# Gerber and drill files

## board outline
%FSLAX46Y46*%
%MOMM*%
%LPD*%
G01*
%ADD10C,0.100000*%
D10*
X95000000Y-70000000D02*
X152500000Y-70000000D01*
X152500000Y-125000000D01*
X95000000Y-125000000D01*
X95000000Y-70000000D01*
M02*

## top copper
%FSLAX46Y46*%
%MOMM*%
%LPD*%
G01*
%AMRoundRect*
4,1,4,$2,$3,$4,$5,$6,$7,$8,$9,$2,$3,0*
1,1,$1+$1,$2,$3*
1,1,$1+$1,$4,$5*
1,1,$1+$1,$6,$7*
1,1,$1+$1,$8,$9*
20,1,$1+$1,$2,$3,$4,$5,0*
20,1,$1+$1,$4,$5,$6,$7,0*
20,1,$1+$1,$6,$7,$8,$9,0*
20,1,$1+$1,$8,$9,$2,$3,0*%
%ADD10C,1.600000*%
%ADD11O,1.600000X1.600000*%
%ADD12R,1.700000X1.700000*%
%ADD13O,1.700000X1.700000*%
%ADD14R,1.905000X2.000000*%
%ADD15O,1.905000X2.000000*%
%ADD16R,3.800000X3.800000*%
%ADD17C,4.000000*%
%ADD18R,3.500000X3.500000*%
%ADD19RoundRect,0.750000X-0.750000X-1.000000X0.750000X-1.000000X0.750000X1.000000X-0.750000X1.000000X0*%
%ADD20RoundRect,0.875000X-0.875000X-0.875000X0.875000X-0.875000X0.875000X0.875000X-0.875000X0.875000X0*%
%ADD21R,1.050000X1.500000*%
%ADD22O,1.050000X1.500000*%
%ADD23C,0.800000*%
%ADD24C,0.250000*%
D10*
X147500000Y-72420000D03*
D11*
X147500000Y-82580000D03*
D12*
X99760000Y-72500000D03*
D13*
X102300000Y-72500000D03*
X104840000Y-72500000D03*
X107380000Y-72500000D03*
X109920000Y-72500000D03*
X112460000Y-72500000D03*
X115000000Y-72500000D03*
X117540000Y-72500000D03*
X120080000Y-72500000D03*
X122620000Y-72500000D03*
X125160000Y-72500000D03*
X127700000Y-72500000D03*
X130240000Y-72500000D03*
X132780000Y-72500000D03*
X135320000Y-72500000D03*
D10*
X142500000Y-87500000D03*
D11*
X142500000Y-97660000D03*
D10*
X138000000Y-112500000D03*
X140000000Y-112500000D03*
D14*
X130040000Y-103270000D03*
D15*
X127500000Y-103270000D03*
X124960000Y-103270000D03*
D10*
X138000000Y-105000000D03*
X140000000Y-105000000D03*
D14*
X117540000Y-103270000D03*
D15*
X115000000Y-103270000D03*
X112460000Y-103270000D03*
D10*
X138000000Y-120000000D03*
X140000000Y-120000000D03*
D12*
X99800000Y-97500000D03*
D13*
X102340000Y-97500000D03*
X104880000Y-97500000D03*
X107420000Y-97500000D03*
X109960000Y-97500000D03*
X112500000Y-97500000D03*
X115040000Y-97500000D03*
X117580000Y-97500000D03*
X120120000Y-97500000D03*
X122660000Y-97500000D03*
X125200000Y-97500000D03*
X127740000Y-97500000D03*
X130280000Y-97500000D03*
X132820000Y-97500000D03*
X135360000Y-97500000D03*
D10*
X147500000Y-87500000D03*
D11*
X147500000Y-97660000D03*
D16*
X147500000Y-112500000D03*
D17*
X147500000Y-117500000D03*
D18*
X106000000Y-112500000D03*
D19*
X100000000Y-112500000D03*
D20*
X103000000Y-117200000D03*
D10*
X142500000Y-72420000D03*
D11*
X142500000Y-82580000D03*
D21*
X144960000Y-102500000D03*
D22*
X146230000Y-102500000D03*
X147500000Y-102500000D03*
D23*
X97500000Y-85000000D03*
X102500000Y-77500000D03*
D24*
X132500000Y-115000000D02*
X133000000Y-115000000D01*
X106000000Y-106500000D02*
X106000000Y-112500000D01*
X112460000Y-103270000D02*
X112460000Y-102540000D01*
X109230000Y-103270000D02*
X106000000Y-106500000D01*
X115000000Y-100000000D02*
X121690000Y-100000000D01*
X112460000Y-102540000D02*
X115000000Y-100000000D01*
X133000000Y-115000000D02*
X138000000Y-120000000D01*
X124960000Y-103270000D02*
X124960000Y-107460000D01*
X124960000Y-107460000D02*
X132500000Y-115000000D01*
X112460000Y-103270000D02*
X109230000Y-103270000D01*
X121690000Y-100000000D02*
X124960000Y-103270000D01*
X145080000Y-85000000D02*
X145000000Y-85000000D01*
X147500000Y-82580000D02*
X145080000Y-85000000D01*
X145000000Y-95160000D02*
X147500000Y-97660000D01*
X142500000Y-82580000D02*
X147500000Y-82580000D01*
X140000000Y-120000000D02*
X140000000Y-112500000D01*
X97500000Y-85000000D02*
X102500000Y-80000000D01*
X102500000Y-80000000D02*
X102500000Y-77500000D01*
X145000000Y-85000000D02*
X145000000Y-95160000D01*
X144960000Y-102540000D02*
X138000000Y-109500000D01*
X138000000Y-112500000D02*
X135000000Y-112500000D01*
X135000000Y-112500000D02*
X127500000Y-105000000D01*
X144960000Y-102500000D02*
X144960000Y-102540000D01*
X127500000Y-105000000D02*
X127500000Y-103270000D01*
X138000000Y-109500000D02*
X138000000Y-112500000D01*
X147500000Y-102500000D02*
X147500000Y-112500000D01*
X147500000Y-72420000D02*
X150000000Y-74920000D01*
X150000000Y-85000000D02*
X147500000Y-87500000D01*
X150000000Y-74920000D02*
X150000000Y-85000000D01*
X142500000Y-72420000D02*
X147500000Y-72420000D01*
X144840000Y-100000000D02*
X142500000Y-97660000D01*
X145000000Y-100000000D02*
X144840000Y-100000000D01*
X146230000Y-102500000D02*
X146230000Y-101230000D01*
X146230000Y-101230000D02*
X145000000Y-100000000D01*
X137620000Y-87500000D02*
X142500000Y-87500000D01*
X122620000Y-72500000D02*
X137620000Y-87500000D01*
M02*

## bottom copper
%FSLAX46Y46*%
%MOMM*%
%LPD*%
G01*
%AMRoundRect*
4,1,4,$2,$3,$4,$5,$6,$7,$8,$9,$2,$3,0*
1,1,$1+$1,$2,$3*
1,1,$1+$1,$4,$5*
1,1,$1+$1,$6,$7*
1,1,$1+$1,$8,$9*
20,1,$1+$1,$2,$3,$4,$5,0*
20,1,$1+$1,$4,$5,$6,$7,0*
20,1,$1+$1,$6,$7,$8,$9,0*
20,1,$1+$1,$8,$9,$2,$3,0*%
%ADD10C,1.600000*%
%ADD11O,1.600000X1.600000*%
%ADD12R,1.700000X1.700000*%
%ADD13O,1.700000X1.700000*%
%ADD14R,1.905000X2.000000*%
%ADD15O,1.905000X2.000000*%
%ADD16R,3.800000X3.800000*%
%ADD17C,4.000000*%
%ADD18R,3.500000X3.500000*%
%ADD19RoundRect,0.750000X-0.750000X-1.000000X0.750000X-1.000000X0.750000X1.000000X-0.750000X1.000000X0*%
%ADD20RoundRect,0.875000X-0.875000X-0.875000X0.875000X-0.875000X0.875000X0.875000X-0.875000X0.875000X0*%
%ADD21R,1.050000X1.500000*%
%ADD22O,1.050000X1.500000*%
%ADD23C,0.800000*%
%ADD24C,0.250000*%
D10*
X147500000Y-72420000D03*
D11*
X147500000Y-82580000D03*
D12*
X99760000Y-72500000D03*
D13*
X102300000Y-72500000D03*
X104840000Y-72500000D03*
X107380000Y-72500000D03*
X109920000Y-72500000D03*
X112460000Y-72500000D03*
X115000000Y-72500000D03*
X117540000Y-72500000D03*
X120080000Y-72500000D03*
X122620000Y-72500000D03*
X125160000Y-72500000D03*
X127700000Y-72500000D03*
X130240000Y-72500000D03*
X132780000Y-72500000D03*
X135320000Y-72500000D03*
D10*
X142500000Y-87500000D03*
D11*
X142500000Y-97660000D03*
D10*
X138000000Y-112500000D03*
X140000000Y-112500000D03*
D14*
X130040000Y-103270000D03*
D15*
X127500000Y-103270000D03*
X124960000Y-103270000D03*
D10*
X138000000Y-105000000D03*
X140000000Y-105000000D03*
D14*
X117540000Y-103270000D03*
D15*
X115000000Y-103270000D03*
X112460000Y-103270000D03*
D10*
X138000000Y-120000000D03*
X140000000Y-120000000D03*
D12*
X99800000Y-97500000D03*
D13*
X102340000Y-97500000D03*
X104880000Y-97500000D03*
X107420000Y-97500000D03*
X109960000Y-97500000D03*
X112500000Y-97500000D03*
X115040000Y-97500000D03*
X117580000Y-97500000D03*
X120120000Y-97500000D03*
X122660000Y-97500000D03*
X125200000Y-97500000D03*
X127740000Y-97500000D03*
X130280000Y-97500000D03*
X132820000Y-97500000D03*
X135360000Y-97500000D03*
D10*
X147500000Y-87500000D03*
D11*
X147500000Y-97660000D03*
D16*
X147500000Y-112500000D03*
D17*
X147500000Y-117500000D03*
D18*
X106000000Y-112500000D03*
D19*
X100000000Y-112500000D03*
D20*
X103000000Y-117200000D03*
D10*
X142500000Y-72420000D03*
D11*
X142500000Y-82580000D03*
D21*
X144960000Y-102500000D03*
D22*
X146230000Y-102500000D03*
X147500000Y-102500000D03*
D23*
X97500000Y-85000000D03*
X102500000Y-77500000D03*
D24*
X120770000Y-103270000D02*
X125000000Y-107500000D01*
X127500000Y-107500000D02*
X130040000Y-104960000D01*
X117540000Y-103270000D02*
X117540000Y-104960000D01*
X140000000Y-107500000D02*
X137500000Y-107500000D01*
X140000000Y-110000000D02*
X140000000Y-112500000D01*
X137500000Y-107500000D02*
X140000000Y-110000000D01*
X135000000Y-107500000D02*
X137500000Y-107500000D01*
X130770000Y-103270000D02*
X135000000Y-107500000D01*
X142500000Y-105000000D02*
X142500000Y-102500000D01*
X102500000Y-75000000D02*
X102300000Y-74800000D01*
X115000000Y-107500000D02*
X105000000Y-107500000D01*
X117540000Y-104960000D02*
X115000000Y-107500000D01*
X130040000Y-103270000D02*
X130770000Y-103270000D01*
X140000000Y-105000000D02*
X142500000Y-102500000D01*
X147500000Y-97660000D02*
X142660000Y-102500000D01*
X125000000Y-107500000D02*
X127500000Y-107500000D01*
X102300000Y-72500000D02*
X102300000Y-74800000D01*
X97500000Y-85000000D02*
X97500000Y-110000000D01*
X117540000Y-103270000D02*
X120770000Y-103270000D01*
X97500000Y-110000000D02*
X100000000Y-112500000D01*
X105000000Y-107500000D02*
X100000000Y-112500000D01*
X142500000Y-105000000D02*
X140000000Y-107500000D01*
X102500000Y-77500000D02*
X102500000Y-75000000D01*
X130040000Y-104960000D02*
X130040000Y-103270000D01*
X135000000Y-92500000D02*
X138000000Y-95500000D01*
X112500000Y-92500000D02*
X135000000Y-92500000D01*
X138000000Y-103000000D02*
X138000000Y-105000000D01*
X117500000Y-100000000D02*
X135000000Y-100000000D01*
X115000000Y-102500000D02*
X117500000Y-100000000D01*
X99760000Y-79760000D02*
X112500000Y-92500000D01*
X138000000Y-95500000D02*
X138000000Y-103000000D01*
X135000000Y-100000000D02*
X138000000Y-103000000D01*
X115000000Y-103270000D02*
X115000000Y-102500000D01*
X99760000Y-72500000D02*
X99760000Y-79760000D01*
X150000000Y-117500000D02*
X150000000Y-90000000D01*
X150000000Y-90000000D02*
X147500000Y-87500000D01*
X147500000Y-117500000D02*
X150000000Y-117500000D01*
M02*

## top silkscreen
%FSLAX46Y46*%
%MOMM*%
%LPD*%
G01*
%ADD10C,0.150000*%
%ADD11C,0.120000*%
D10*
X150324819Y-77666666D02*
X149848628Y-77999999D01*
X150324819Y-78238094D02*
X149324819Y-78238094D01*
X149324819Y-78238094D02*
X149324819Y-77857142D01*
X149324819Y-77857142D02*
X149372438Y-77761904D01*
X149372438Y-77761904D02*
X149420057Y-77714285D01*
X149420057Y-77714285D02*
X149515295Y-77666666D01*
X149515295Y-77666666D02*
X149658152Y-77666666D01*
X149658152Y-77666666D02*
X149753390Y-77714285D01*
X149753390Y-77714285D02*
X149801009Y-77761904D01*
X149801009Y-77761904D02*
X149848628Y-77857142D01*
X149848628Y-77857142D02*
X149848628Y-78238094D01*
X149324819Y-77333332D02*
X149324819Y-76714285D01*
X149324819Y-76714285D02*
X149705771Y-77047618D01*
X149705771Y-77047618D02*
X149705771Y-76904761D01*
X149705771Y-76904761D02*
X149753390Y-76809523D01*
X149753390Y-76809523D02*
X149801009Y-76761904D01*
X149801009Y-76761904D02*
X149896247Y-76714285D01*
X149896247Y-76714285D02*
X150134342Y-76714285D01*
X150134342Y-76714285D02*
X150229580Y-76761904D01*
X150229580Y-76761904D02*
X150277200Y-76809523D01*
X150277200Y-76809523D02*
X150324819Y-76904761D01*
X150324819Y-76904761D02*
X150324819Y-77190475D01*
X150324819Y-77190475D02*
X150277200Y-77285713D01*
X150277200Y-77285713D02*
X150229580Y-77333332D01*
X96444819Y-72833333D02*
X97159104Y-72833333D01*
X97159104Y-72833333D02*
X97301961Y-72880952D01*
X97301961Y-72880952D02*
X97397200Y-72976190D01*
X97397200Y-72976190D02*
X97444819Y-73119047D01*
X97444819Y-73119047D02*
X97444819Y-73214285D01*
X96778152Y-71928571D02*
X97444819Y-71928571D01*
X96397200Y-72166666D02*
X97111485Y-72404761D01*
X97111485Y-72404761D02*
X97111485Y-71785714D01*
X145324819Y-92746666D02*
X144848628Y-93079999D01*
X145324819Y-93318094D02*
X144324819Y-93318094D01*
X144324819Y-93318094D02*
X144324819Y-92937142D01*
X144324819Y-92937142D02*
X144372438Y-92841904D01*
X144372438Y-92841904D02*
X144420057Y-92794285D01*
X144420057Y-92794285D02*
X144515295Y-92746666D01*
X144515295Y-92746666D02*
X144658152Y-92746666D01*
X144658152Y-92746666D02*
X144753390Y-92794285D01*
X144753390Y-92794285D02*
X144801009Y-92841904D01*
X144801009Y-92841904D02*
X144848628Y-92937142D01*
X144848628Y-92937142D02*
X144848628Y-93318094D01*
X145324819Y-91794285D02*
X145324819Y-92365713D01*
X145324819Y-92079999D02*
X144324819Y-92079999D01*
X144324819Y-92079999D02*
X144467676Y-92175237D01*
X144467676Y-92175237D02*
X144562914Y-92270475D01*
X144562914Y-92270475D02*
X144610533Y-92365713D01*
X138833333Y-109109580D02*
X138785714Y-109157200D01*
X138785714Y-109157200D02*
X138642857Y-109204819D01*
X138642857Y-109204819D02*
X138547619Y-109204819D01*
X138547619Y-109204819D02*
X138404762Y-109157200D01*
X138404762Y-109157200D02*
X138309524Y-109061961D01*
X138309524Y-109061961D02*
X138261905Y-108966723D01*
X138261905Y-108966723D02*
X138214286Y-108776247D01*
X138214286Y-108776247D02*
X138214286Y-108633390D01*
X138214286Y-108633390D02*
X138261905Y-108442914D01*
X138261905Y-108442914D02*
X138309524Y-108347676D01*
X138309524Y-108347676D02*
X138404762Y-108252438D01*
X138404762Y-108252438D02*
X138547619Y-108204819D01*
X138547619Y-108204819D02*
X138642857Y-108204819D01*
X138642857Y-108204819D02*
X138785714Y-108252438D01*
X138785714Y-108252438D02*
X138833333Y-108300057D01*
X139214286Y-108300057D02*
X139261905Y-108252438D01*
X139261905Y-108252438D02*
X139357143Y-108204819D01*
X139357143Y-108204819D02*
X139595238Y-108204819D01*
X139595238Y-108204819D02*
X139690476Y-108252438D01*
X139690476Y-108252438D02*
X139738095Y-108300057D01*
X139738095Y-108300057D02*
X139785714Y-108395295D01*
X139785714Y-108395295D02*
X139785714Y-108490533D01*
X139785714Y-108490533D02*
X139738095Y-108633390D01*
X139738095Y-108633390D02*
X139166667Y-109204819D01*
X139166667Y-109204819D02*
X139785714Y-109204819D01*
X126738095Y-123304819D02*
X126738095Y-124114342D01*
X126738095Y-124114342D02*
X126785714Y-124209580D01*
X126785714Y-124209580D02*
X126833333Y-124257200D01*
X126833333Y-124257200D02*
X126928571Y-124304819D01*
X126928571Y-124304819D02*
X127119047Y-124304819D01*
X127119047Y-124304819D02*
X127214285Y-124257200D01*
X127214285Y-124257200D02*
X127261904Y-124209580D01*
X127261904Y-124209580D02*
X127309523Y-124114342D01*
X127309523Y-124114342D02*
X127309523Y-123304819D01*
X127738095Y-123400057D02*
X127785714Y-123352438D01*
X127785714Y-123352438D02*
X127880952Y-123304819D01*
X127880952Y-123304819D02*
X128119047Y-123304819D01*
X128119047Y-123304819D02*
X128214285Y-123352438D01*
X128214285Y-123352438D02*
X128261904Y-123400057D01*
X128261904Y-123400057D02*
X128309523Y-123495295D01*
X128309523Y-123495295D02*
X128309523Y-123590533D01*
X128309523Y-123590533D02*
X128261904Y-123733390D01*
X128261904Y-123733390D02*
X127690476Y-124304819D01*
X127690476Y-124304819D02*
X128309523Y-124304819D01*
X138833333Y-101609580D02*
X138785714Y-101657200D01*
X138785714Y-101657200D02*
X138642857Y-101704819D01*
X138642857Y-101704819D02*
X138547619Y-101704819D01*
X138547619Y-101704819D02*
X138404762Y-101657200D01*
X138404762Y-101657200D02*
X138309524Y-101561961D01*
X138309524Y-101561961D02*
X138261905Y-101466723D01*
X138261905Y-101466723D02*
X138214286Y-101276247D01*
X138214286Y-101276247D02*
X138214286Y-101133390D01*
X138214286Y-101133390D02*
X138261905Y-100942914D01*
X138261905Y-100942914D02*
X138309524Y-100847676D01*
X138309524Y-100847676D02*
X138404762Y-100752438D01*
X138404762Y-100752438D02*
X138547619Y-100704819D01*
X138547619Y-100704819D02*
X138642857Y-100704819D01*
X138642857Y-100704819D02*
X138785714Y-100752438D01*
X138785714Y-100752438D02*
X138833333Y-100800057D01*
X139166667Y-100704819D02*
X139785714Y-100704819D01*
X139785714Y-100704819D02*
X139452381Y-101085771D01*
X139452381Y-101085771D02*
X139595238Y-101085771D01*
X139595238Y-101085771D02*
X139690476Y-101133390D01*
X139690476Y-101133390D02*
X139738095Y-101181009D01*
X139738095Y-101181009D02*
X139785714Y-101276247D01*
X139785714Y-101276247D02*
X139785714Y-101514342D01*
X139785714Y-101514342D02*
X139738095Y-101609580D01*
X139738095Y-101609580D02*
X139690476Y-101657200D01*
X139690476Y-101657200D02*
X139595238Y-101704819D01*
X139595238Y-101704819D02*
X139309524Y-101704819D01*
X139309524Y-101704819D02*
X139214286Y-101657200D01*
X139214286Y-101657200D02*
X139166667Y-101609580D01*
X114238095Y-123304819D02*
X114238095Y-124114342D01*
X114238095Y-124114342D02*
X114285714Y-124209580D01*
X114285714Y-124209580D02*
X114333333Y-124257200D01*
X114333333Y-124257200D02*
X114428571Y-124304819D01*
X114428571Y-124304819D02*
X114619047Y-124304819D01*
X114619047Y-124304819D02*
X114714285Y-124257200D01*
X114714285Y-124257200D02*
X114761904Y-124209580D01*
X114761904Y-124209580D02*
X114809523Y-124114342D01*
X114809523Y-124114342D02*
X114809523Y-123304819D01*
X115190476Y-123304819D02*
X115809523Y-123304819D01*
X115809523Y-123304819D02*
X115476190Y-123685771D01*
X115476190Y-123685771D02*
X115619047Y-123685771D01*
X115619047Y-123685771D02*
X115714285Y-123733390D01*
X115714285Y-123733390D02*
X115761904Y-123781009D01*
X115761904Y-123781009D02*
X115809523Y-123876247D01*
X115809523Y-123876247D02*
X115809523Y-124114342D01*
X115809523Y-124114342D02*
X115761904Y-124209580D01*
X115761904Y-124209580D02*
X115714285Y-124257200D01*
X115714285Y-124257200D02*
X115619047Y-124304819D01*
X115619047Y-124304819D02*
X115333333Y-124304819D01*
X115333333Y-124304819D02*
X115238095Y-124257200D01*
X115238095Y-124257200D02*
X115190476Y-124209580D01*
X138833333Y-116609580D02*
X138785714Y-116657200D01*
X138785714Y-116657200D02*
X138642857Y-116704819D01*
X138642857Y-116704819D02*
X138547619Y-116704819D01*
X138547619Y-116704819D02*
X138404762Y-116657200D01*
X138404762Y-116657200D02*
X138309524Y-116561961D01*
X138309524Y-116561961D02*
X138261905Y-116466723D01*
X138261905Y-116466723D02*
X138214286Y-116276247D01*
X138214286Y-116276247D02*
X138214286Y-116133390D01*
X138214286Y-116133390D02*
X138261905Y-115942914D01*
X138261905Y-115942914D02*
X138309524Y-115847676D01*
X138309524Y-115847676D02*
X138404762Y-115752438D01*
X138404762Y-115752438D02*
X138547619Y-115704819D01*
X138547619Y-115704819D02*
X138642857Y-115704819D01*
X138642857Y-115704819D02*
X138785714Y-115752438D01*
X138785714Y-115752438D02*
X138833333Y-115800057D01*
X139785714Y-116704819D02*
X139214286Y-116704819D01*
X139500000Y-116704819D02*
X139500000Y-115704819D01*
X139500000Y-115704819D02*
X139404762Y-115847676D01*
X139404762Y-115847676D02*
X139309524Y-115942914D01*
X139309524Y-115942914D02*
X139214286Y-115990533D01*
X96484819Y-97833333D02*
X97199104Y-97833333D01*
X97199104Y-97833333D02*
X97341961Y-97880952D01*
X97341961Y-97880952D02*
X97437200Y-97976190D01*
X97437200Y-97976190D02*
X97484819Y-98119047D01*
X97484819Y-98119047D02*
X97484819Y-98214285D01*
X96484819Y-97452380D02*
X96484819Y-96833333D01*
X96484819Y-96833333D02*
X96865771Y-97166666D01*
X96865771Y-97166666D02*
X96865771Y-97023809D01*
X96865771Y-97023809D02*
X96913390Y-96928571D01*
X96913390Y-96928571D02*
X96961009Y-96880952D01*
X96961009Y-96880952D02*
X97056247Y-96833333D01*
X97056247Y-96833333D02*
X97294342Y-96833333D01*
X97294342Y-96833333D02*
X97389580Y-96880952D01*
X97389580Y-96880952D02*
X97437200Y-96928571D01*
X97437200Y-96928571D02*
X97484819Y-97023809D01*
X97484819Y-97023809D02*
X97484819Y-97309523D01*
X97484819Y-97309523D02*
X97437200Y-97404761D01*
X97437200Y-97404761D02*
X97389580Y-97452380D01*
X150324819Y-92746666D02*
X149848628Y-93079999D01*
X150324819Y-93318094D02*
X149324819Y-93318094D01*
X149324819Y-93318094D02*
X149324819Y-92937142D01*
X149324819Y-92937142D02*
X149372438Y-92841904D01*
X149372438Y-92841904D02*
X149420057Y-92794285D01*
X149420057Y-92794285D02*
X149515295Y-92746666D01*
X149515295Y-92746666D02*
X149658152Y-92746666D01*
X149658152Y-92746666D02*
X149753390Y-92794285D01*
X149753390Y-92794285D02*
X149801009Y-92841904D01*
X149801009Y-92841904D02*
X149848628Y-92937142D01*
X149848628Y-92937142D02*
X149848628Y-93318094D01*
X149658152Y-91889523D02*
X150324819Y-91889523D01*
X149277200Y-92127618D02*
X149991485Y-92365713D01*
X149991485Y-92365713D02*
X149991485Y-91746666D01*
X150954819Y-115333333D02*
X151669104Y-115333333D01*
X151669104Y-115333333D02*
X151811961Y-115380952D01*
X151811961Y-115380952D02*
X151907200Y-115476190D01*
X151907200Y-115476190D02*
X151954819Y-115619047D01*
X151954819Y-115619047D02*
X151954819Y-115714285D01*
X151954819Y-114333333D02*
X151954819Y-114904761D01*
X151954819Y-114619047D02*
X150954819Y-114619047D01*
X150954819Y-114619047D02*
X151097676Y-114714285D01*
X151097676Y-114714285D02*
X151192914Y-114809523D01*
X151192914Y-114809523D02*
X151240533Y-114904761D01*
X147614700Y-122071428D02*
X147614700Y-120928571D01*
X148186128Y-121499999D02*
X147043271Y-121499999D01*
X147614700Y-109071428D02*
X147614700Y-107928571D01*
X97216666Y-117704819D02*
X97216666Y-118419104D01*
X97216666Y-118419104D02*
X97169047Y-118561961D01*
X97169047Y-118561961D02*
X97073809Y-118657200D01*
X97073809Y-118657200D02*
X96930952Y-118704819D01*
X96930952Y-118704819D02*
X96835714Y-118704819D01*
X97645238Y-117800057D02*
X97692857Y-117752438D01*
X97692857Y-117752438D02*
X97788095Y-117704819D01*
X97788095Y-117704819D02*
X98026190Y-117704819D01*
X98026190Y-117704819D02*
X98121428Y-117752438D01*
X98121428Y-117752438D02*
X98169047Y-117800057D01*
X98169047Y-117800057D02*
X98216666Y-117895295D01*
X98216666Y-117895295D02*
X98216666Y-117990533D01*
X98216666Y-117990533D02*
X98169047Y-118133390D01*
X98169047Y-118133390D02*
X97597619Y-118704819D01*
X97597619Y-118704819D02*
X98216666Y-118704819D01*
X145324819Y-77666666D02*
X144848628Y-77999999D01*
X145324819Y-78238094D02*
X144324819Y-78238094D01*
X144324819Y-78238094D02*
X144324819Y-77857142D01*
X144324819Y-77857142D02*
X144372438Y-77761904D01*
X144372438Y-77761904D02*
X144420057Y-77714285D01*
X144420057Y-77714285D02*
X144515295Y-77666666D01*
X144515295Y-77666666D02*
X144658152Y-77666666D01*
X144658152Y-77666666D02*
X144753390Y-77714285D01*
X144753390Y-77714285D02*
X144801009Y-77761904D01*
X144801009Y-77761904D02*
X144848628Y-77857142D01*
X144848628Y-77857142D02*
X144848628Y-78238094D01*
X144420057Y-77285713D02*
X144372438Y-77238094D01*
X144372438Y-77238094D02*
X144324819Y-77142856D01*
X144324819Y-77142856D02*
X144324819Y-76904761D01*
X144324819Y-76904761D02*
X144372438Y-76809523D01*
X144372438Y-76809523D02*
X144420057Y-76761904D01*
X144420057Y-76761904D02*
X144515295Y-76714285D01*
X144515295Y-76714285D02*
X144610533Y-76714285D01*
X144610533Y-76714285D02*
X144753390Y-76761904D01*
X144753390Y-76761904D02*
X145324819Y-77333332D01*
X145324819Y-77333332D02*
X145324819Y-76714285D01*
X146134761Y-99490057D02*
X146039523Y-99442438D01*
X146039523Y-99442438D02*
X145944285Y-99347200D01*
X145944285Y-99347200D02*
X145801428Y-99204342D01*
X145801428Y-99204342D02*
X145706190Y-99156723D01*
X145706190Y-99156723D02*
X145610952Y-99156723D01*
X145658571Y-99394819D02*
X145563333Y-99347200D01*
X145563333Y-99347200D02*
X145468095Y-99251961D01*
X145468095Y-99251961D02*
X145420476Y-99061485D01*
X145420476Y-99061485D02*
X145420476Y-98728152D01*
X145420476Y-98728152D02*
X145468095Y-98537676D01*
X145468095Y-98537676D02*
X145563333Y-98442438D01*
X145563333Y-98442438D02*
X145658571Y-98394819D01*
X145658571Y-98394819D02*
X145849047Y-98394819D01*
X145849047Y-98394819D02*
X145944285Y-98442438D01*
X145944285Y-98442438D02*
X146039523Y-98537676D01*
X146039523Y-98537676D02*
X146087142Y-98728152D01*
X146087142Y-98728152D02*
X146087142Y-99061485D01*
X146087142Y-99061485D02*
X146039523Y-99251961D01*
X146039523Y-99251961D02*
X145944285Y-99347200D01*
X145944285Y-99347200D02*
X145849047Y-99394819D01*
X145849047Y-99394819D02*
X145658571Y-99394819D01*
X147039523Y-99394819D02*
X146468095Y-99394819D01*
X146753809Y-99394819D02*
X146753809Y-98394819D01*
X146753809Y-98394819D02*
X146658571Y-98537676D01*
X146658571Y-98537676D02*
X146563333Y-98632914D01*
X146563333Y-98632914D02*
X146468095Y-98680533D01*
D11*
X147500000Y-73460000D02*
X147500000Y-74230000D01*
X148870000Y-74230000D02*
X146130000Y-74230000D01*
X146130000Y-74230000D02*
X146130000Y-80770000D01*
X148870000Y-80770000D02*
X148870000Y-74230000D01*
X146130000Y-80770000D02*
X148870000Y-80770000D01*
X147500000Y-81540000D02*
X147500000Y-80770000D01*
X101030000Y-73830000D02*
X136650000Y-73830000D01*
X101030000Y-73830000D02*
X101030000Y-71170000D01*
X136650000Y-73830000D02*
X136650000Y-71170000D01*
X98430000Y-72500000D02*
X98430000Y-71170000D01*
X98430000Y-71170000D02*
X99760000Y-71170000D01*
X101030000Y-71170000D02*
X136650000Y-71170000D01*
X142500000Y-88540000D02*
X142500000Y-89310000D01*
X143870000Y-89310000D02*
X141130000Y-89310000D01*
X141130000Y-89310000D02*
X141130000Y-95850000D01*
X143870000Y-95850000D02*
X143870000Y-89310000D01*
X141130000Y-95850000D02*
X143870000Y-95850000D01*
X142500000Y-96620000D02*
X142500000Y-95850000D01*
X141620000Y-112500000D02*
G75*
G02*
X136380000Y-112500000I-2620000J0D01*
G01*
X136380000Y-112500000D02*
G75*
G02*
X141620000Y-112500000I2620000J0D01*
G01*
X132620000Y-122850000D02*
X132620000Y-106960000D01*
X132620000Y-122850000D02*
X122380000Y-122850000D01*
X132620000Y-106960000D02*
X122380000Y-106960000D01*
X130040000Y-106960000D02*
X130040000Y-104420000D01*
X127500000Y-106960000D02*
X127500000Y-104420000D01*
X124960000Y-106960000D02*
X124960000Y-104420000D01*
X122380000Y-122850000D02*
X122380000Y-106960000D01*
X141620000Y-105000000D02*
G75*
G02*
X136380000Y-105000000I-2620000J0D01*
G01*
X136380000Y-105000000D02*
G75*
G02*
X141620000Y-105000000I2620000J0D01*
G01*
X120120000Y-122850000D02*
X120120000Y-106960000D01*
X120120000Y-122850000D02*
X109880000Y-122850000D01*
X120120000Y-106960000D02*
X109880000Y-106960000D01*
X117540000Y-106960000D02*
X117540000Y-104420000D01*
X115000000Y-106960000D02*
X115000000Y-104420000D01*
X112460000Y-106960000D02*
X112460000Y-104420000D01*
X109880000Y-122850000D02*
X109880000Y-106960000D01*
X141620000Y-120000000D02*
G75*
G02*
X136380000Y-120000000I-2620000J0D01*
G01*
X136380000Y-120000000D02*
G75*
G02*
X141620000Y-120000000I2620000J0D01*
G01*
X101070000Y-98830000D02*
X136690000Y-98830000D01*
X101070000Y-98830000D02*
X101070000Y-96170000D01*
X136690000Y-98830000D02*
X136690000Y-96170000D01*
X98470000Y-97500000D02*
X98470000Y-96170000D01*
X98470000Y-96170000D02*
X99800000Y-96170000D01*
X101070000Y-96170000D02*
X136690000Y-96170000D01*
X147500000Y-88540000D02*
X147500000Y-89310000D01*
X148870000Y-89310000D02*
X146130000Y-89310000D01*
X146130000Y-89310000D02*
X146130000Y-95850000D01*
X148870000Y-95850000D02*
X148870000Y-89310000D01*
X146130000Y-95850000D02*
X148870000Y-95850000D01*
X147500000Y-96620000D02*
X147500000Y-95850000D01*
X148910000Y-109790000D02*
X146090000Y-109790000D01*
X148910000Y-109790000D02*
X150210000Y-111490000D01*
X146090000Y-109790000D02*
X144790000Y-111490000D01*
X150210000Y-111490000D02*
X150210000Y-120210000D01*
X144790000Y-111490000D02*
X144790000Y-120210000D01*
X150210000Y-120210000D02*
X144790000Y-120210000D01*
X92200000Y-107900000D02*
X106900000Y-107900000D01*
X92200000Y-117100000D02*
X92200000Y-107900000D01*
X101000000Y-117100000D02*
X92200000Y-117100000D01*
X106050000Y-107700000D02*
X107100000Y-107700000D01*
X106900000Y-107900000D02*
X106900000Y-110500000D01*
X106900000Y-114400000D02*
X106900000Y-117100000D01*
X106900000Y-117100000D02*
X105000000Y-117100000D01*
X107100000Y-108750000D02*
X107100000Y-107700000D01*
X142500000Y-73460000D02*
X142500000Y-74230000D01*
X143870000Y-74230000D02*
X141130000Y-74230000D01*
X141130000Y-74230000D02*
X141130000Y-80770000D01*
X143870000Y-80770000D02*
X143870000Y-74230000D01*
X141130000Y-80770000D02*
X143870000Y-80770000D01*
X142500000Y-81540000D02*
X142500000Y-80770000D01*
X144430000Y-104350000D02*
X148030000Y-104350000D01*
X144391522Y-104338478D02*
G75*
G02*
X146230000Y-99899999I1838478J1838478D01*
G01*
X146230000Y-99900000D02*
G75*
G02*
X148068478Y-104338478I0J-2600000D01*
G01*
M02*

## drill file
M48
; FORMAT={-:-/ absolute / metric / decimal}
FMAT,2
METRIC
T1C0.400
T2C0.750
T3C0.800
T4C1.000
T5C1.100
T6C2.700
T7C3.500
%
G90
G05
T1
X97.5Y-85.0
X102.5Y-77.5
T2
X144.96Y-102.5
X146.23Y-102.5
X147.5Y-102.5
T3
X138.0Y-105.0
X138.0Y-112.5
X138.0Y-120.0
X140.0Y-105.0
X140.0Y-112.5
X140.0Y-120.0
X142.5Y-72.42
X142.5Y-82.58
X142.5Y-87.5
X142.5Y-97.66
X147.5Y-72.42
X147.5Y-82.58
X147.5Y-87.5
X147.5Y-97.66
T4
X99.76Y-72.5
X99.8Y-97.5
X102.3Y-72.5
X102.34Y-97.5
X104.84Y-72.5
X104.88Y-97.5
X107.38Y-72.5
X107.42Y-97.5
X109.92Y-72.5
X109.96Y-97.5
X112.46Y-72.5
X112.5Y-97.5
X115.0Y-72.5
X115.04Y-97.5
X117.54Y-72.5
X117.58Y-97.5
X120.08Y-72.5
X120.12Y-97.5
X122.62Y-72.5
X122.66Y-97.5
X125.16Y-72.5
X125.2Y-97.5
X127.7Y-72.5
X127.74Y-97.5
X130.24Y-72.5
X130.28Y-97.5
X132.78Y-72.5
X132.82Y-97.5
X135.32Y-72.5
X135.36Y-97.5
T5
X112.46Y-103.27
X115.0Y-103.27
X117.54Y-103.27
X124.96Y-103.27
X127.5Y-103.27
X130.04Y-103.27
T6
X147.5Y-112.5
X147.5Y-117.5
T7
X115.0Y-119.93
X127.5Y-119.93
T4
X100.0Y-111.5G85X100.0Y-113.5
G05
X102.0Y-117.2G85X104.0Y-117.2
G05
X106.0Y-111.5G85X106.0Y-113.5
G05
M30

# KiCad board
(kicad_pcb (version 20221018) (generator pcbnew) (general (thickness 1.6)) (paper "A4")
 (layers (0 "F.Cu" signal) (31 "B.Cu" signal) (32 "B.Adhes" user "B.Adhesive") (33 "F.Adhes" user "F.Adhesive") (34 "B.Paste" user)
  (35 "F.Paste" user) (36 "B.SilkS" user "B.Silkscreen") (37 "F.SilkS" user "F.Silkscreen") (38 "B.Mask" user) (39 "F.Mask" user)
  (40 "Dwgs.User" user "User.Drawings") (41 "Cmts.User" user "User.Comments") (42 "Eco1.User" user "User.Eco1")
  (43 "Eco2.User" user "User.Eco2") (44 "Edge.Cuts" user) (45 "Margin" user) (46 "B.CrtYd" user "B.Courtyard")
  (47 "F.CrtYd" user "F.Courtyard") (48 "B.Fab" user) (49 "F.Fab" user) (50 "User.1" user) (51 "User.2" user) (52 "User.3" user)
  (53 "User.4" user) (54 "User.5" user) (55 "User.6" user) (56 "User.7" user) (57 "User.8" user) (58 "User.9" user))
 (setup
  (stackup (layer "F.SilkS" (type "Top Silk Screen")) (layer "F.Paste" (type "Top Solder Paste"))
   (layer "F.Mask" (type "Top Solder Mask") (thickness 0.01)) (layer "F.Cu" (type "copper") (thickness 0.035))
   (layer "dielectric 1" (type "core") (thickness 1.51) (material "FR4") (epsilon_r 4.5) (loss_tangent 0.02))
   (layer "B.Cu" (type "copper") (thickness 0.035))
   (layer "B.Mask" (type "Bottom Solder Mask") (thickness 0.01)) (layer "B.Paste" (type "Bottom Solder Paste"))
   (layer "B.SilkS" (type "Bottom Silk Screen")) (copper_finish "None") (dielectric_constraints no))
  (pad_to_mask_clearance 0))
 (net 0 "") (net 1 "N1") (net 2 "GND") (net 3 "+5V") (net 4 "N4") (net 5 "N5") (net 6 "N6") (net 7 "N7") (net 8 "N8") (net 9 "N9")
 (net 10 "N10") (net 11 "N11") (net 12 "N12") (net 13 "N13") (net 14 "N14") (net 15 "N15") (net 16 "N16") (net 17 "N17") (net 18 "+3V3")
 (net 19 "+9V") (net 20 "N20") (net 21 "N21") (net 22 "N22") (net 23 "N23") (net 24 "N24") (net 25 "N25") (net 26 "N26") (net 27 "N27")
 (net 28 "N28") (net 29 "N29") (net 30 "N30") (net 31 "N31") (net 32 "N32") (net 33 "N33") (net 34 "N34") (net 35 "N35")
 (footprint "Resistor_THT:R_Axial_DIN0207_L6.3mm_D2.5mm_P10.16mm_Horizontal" (layer "F.Cu") (at 147.5 72.42 -90)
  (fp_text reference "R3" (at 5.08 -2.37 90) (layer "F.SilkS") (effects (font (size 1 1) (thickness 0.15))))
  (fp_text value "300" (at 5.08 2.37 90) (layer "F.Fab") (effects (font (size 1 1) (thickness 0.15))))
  (fp_line (start 1.04 0) (end 1.81 0) (stroke (width 0.12) (type solid)) (layer "F.SilkS"))
  (fp_line (start 1.81 -1.37) (end 1.81 1.37) (stroke (width 0.12) (type solid)) (layer "F.SilkS"))
  (fp_line (start 1.81 1.37) (end 8.35 1.37) (stroke (width 0.12) (type solid)) (layer "F.SilkS"))
  (fp_line (start 8.35 -1.37) (end 1.81 -1.37) (stroke (width 0.12) (type solid)) (layer "F.SilkS"))
  (fp_line (start 8.35 1.37) (end 8.35 -1.37) (stroke (width 0.12) (type solid)) (layer "F.SilkS"))
  (fp_line (start 9.12 0) (end 8.35 0) (stroke (width 0.12) (type solid)) (layer "F.SilkS"))
  (pad "1" thru_hole circle (at 0 0 270) (size 1.6 1.6) (drill 0.8) (layers "*.Cu" "*.Mask") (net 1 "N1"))
  (pad "2" thru_hole oval (at 10.16 0 270) (size 1.6 1.6) (drill 0.8) (layers "*.Cu" "*.Mask") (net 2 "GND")))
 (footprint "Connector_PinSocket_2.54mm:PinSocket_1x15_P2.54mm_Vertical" (layer "F.Cu") (at 99.76 72.5 90)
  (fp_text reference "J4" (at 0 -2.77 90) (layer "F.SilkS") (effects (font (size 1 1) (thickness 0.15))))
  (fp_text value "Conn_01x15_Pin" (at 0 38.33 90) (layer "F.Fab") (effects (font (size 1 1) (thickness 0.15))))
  (fp_line (start -1.33 1.27) (end -1.33 36.89) (stroke (width 0.12) (type solid)) (layer "F.SilkS"))
  (fp_line (start -1.33 1.27) (end 1.33 1.27) (stroke (width 0.12) (type solid)) (layer "F.SilkS"))
  (fp_line (start -1.33 36.89) (end 1.33 36.89) (stroke (width 0.12) (type solid)) (layer "F.SilkS"))
  (fp_line (start 0 -1.33) (end 1.33 -1.33) (stroke (width 0.12) (type solid)) (layer "F.SilkS"))
  (fp_line (start 1.33 -1.33) (end 1.33 0) (stroke (width 0.12) (type solid)) (layer "F.SilkS"))
  (fp_line (start 1.33 1.27) (end 1.33 36.89) (stroke (width 0.12) (type solid)) (layer "F.SilkS"))
  (pad "1" thru_hole rect (at 0 0 90) (size 1.7 1.7) (drill 1) (layers "*.Cu" "*.Mask") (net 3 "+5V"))
  (pad "2" thru_hole oval (at 0 2.54 90) (size 1.7 1.7) (drill 1) (layers "*.Cu" "*.Mask") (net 2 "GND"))
  (pad "3" thru_hole oval (at 0 5.08 90) (size 1.7 1.7) (drill 1) (layers "*.Cu" "*.Mask") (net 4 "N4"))
  (pad "4" thru_hole oval (at 0 7.62 90) (size 1.7 1.7) (drill 1) (layers "*.Cu" "*.Mask") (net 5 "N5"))
  (pad "5" thru_hole oval (at 0 10.16 90) (size 1.7 1.7) (drill 1) (layers "*.Cu" "*.Mask") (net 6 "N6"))
  (pad "6" thru_hole oval (at 0 12.7 90) (size 1.7 1.7) (drill 1) (layers "*.Cu" "*.Mask") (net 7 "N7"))
  (pad "7" thru_hole oval (at 0 15.24 90) (size 1.7 1.7) (drill 1) (layers "*.Cu" "*.Mask") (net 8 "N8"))
  (pad "8" thru_hole oval (at 0 17.78 90) (size 1.7 1.7) (drill 1) (layers "*.Cu" "*.Mask") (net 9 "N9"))
  (pad "9" thru_hole oval (at 0 20.32 90) (size 1.7 1.7) (drill 1) (layers "*.Cu" "*.Mask") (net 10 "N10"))
  (pad "10" thru_hole oval (at 0 22.86 90) (size 1.7 1.7) (drill 1) (layers "*.Cu" "*.Mask") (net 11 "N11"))
  (pad "11" thru_hole oval (at 0 25.4 90) (size 1.7 1.7) (drill 1) (layers "*.Cu" "*.Mask") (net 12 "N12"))
  (pad "12" thru_hole oval (at 0 27.94 90) (size 1.7 1.7) (drill 1) (layers "*.Cu" "*.Mask") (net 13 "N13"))
  (pad "13" thru_hole oval (at 0 30.48 90) (size 1.7 1.7) (drill 1) (layers "*.Cu" "*.Mask") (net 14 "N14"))
  (pad "14" thru_hole oval (at 0 33.02 90) (size 1.7 1.7) (drill 1) (layers "*.Cu" "*.Mask") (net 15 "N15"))
  (pad "15" thru_hole oval (at 0 35.56 90) (size 1.7 1.7) (drill 1) (layers "*.Cu" "*.Mask") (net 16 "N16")))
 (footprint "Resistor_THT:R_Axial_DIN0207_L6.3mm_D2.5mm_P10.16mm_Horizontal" (layer "F.Cu") (at 142.5 87.5 -90)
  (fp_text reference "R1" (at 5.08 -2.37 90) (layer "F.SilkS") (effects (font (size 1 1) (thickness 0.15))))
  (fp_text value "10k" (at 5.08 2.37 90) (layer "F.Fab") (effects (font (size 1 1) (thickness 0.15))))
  (fp_line (start 1.04 0) (end 1.81 0) (stroke (width 0.12) (type solid)) (layer "F.SilkS"))
  (fp_line (start 1.81 -1.37) (end 1.81 1.37) (stroke (width 0.12) (type solid)) (layer "F.SilkS"))
  (fp_line (start 1.81 1.37) (end 8.35 1.37) (stroke (width 0.12) (type solid)) (layer "F.SilkS"))
  (fp_line (start 8.35 -1.37) (end 1.81 -1.37) (stroke (width 0.12) (type solid)) (layer "F.SilkS"))
  (fp_line (start 8.35 1.37) (end 8.35 -1.37) (stroke (width 0.12) (type solid)) (layer "F.SilkS"))
  (fp_line (start 9.12 0) (end 8.35 0) (stroke (width 0.12) (type solid)) (layer "F.SilkS"))
  (pad "1" thru_hole circle (at 0 0 270) (size 1.6 1.6) (drill 0.8) (layers "*.Cu" "*.Mask") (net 11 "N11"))
  (pad "2" thru_hole oval (at 10.16 0 270) (size 1.6 1.6) (drill 0.8) (layers "*.Cu" "*.Mask") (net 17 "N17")))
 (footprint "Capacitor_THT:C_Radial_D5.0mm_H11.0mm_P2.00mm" (layer "F.Cu") (at 138 112.5)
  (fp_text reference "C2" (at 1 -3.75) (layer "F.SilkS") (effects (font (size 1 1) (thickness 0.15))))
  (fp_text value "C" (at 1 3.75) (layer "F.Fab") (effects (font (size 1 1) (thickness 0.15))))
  (fp_circle (center 1 0) (end 3.62 0) (stroke (width 0.12) (type solid)) (fill none) (layer "F.SilkS"))
  (pad "1" thru_hole circle (at 0 0) (size 1.6 1.6) (drill 0.8) (layers "*.Cu" "*.Mask") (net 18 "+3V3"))
  (pad "2" thru_hole circle (at 2 0) (size 1.6 1.6) (drill 0.8) (layers "*.Cu" "*.Mask") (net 2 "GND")))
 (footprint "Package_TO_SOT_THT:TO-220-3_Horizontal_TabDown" (layer "F.Cu") (at 130.04 103.27 180)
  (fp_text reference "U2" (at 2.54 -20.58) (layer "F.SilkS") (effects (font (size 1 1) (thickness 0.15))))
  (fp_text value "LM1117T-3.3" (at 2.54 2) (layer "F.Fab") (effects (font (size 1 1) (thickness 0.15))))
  (fp_line (start -2.58 -19.58) (end -2.58 -3.69) (stroke (width 0.12) (type solid)) (layer "F.SilkS"))
  (fp_line (start -2.58 -19.58) (end 7.66 -19.58) (stroke (width 0.12) (type solid)) (layer "F.SilkS"))
  (fp_line (start -2.58 -3.69) (end 7.66 -3.69) (stroke (width 0.12) (type solid)) (layer "F.SilkS"))
  (fp_line (start 0 -3.69) (end 0 -1.15) (stroke (width 0.12) (type solid)) (layer "F.SilkS"))
  (fp_line (start 2.54 -3.69) (end 2.54 -1.15) (stroke (width 0.12) (type solid)) (layer "F.SilkS"))
  (fp_line (start 5.08 -3.69) (end 5.08 -1.15) (stroke (width 0.12) (type solid)) (layer "F.SilkS"))
  (fp_line (start 7.66 -19.58) (end 7.66 -3.69) (stroke (width 0.12) (type solid)) (layer "F.SilkS"))
  (pad "" np_thru_hole oval (at 2.54 -16.66 180) (size 3.5 3.5) (drill 3.5) (layers "*.Cu" "*.Mask"))
  (pad "1" thru_hole rect (at 0 0 180) (size 1.905 2) (drill 1.1) (layers "*.Cu" "*.Mask") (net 2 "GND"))
  (pad "2" thru_hole oval (at 2.54 0 180) (size 1.905 2) (drill 1.1) (layers "*.Cu" "*.Mask") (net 18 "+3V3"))
  (pad "3" thru_hole oval (at 5.08 0 180) (size 1.905 2) (drill 1.1) (layers "*.Cu" "*.Mask") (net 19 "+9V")))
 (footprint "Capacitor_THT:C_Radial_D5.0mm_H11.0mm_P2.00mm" (layer "F.Cu") (at 138 105)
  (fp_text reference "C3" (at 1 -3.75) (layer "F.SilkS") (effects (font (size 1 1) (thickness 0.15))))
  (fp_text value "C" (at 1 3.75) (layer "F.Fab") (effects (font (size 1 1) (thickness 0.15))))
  (fp_circle (center 1 0) (end 3.62 0) (stroke (width 0.12) (type solid)) (fill none) (layer "F.SilkS"))
  (pad "1" thru_hole circle (at 0 0) (size 1.6 1.6) (drill 0.8) (layers "*.Cu" "*.Mask") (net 3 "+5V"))
  (pad "2" thru_hole circle (at 2 0) (size 1.6 1.6) (drill 0.8) (layers "*.Cu" "*.Mask") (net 2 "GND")))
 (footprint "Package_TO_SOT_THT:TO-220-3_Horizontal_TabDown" (layer "F.Cu") (at 117.54 103.27 180)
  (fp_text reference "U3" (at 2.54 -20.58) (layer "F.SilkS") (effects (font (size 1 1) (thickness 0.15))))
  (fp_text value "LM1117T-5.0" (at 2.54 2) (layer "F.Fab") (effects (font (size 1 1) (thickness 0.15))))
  (fp_line (start -2.58 -19.58) (end -2.58 -3.69) (stroke (width 0.12) (type solid)) (layer "F.SilkS"))
  (fp_line (start -2.58 -19.58) (end 7.66 -19.58) (stroke (width 0.12) (type solid)) (layer "F.SilkS"))
  (fp_line (start -2.58 -3.69) (end 7.66 -3.69) (stroke (width 0.12) (type solid)) (layer "F.SilkS"))
  (fp_line (start 0 -3.69) (end 0 -1.15) (stroke (width 0.12) (type solid)) (layer "F.SilkS"))
  (fp_line (start 2.54 -3.69) (end 2.54 -1.15) (stroke (width 0.12) (type solid)) (layer "F.SilkS"))
  (fp_line (start 5.08 -3.69) (end 5.08 -1.15) (stroke (width 0.12) (type solid)) (layer "F.SilkS"))
  (fp_line (start 7.66 -19.58) (end 7.66 -3.69) (stroke (width 0.12) (type solid)) (layer "F.SilkS"))
  (pad "" np_thru_hole oval (at 2.54 -16.66 180) (size 3.5 3.5) (drill 3.5) (layers "*.Cu" "*.Mask"))
  (pad "1" thru_hole rect (at 0 0 180) (size 1.905 2) (drill 1.1) (layers "*.Cu" "*.Mask") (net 2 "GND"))
  (pad "2" thru_hole oval (at 2.54 0 180) (size 1.905 2) (drill 1.1) (layers "*.Cu" "*.Mask") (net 3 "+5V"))
  (pad "3" thru_hole oval (at 5.08 0 180) (size 1.905 2) (drill 1.1) (layers "*.Cu" "*.Mask") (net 19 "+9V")))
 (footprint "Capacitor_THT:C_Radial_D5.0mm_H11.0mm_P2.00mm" (layer "F.Cu") (at 138 120)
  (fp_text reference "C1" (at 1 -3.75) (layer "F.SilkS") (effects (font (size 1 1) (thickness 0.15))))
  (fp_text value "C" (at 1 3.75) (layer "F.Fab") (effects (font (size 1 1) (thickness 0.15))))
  (fp_circle (center 1 0) (end 3.62 0) (stroke (width 0.12) (type solid)) (fill none) (layer "F.SilkS"))
  (pad "1" thru_hole circle (at 0 0) (size 1.6 1.6) (drill 0.8) (layers "*.Cu" "*.Mask") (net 19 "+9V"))
  (pad "2" thru_hole circle (at 2 0) (size 1.6 1.6) (drill 0.8) (layers "*.Cu" "*.Mask") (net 2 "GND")))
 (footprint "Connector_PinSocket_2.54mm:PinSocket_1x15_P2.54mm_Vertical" (layer "F.Cu") (at 99.8 97.5 90)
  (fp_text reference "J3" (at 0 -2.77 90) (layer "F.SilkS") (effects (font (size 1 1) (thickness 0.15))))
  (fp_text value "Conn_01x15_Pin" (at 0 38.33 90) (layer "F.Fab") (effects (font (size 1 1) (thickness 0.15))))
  (fp_line (start -1.33 1.27) (end -1.33 36.89) (stroke (width 0.12) (type solid)) (layer "F.SilkS"))
  (fp_line (start -1.33 1.27) (end 1.33 1.27) (stroke (width 0.12) (type solid)) (layer "F.SilkS"))
  (fp_line (start -1.33 36.89) (end 1.33 36.89) (stroke (width 0.12) (type solid)) (layer "F.SilkS"))
  (fp_line (start 0 -1.33) (end 1.33 -1.33) (stroke (width 0.12) (type solid)) (layer "F.SilkS"))
  (fp_line (start 1.33 -1.33) (end 1.33 0) (stroke (width 0.12) (type solid)) (layer "F.SilkS"))
  (fp_line (start 1.33 1.27) (end 1.33 36.89) (stroke (width 0.12) (type solid)) (layer "F.SilkS"))
  (pad "1" thru_hole rect (at 0 0 90) (size 1.7 1.7) (drill 1) (layers "*.Cu" "*.Mask") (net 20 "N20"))
  (pad "2" thru_hole oval (at 0 2.54 90) (size 1.7 1.7) (drill 1) (layers "*.Cu" "*.Mask") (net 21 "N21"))
  (pad "3" thru_hole oval (at 0 5.08 90) (size 1.7 1.7) (drill 1) (layers "*.Cu" "*.Mask") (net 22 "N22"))
  (pad "4" thru_hole oval (at 0 7.62 90) (size 1.7 1.7) (drill 1) (layers "*.Cu" "*.Mask") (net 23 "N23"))
  (pad "5" thru_hole oval (at 0 10.16 90) (size 1.7 1.7) (drill 1) (layers "*.Cu" "*.Mask") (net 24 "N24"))
  (pad "6" thru_hole oval (at 0 12.7 90) (size 1.7 1.7) (drill 1) (layers "*.Cu" "*.Mask") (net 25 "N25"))
  (pad "7" thru_hole oval (at 0 15.24 90) (size 1.7 1.7) (drill 1) (layers "*.Cu" "*.Mask") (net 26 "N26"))
  (pad "8" thru_hole oval (at 0 17.78 90) (size 1.7 1.7) (drill 1) (layers "*.Cu" "*.Mask") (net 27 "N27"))
  (pad "9" thru_hole oval (at 0 20.32 90) (size 1.7 1.7) (drill 1) (layers "*.Cu" "*.Mask") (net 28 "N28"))
  (pad "10" thru_hole oval (at 0 22.86 90) (size 1.7 1.7) (drill 1) (layers "*.Cu" "*.Mask") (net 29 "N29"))
  (pad "11" thru_hole oval (at 0 25.4 90) (size 1.7 1.7) (drill 1) (layers "*.Cu" "*.Mask") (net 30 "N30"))
  (pad "12" thru_hole oval (at 0 27.94 90) (size 1.7 1.7) (drill 1) (layers "*.Cu" "*.Mask") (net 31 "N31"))
  (pad "13" thru_hole oval (at 0 30.48 90) (size 1.7 1.7) (drill 1) (layers "*.Cu" "*.Mask") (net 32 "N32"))
  (pad "14" thru_hole oval (at 0 33.02 90) (size 1.7 1.7) (drill 1) (layers "*.Cu" "*.Mask") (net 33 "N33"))
  (pad "15" thru_hole oval (at 0 35.56 90) (size 1.7 1.7) (drill 1) (layers "*.Cu" "*.Mask") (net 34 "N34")))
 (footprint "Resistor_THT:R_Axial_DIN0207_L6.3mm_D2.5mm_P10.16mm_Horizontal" (layer "F.Cu") (at 147.5 87.5 -90)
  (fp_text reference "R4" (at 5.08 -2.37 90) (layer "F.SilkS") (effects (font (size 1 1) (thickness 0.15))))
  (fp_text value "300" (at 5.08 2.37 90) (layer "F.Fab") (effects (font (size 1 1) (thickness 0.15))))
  (fp_line (start 1.04 0) (end 1.81 0) (stroke (width 0.12) (type solid)) (layer "F.SilkS"))
  (fp_line (start 1.81 -1.37) (end 1.81 1.37) (stroke (width 0.12) (type solid)) (layer "F.SilkS"))
  (fp_line (start 1.81 1.37) (end 8.35 1.37) (stroke (width 0.12) (type solid)) (layer "F.SilkS"))
  (fp_line (start 8.35 -1.37) (end 1.81 -1.37) (stroke (width 0.12) (type solid)) (layer "F.SilkS"))
  (fp_line (start 8.35 1.37) (end 8.35 -1.37) (stroke (width 0.12) (type solid)) (layer "F.SilkS"))
  (fp_line (start 9.12 0) (end 8.35 0) (stroke (width 0.12) (type solid)) (layer "F.SilkS"))
  (pad "1" thru_hole circle (at 0 0 270) (size 1.6 1.6) (drill 0.8) (layers "*.Cu" "*.Mask") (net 1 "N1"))
  (pad "2" thru_hole oval (at 10.16 0 270) (size 1.6 1.6) (drill 0.8) (layers "*.Cu" "*.Mask") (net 2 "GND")))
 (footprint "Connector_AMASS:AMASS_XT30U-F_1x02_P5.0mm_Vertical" (layer "F.Cu") (at 147.5 112.5 -90)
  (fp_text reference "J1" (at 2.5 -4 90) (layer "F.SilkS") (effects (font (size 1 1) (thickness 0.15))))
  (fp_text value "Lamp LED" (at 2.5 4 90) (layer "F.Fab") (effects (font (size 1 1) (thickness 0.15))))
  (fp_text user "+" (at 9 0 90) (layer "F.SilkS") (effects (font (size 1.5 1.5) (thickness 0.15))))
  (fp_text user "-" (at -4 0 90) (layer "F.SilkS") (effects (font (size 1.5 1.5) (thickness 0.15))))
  (fp_line (start -2.71 -1.41) (end -2.71 1.41) (stroke (width 0.12) (type solid)) (layer "F.SilkS"))
  (fp_line (start -2.71 -1.41) (end -1.01 -2.71) (stroke (width 0.12) (type solid)) (layer "F.SilkS"))
  (fp_line (start -2.71 1.41) (end -1.01 2.71) (stroke (width 0.12) (type solid)) (layer "F.SilkS"))
  (fp_line (start -1.01 -2.71) (end 7.71 -2.71) (stroke (width 0.12) (type solid)) (layer "F.SilkS"))
  (fp_line (start -1.01 2.71) (end 7.71 2.71) (stroke (width 0.12) (type solid)) (layer "F.SilkS"))
  (fp_line (start 7.71 -2.71) (end 7.71 2.71) (stroke (width 0.12) (type solid)) (layer "F.SilkS"))
  (pad "1" thru_hole rect (at 0 0 270) (size 3.8 3.8) (drill 2.7) (layers "*.Cu" "*.Mask") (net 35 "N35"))
  (pad "2" thru_hole circle (at 5 0 270) (size 4 4) (drill 2.7) (layers "*.Cu" "*.Mask") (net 1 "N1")))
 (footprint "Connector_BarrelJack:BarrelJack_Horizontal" (layer "F.Cu") (at 106 112.5)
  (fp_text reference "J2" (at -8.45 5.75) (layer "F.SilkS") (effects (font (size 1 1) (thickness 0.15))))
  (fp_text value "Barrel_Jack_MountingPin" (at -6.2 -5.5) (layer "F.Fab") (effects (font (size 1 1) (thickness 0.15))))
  (fp_line (start -13.8 -4.6) (end 0.9 -4.6) (stroke (width 0.12) (type solid)) (layer "F.SilkS"))
  (fp_line (start -13.8 4.6) (end -13.8 -4.6) (stroke (width 0.12) (type solid)) (layer "F.SilkS"))
  (fp_line (start -5 4.6) (end -13.8 4.6) (stroke (width 0.12) (type solid)) (layer "F.SilkS"))
  (fp_line (start 0.05 -4.8) (end 1.1 -4.8) (stroke (width 0.12) (type solid)) (layer "F.SilkS"))
  (fp_line (start 0.9 -4.6) (end 0.9 -2) (stroke (width 0.12) (type solid)) (layer "F.SilkS"))
  (fp_line (start 0.9 1.9) (end 0.9 4.6) (stroke (width 0.12) (type solid)) (layer "F.SilkS"))
  (fp_line (start 0.9 4.6) (end -1 4.6) (stroke (width 0.12) (type solid)) (layer "F.SilkS"))
  (fp_line (start 1.1 -3.75) (end 1.1 -4.8) (stroke (width 0.12) (type solid)) (layer "F.SilkS"))
  (pad "1" thru_hole rect (at 0 0) (size 3.5 3.5) (drill oval 1 3) (layers "*.Cu" "*.Mask") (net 19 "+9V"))
  (pad "2" thru_hole roundrect (at -6 0) (size 3 3.5) (drill oval 1 3) (layers "*.Cu" "*.Mask") (roundrect_rratio 0.25) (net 2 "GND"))
  (pad "3" thru_hole roundrect (at -3 4.7) (size 3.5 3.5) (drill oval 3 1) (layers "*.Cu" "*.Mask") (roundrect_rratio 0.25)))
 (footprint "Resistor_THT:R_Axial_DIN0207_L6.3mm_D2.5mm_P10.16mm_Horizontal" (layer "F.Cu") (at 142.5 72.42 -90)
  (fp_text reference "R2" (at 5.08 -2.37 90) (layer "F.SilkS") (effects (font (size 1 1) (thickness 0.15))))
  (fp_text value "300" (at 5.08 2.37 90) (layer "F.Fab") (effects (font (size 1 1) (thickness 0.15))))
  (fp_line (start 1.04 0) (end 1.81 0) (stroke (width 0.12) (type solid)) (layer "F.SilkS"))
  (fp_line (start 1.81 -1.37) (end 1.81 1.37) (stroke (width 0.12) (type solid)) (layer "F.SilkS"))
  (fp_line (start 1.81 1.37) (end 8.35 1.37) (stroke (width 0.12) (type solid)) (layer "F.SilkS"))
  (fp_line (start 8.35 -1.37) (end 1.81 -1.37) (stroke (width 0.12) (type solid)) (layer "F.SilkS"))
  (fp_line (start 8.35 1.37) (end 8.35 -1.37) (stroke (width 0.12) (type solid)) (layer "F.SilkS"))
  (fp_line (start 9.12 0) (end 8.35 0) (stroke (width 0.12) (type solid)) (layer "F.SilkS"))
  (pad "1" thru_hole circle (at 0 0 270) (size 1.6 1.6) (drill 0.8) (layers "*.Cu" "*.Mask") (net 1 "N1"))
  (pad "2" thru_hole oval (at 10.16 0 270) (size 1.6 1.6) (drill 0.8) (layers "*.Cu" "*.Mask") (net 2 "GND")))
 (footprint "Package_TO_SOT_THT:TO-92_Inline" (layer "F.Cu") (at 144.96 102.5)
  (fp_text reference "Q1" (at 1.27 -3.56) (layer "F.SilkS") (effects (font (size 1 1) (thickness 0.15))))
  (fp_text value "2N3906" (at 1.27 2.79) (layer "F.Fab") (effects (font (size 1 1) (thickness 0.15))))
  (fp_line (start -0.53 1.85) (end 3.07 1.85) (stroke (width 0.12) (type solid)) (layer "F.SilkS"))
  (fp_arc (start -0.568478 1.838478) (mid -1.132087 -0.994977) (end 1.27 -2.6) (stroke (width 0.12) (type solid)) (layer "F.SilkS"))
  (fp_arc (start 1.27 -2.6) (mid 3.672087 -0.994977) (end 3.108478 1.838478) (stroke (width 0.12) (type solid)) (layer "F.SilkS"))
  (pad "1" thru_hole rect (at 0 0) (size 1.05 1.5) (drill 0.75) (layers "*.Cu" "*.Mask") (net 18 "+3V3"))
  (pad "2" thru_hole oval (at 1.27 0) (size 1.05 1.5) (drill 0.75) (layers "*.Cu" "*.Mask") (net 17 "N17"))
  (pad "3" thru_hole oval (at 2.54 0) (size 1.05 1.5) (drill 0.75) (layers "*.Cu" "*.Mask") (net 35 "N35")))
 (gr_rect (start 95 70) (end 152.5 125) (stroke (width 0.1) (type default)) (fill none) (layer "Edge.Cuts"))
 (segment (start 132.5 115) (end 133 115) (width 0.25) (layer "F.Cu") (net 19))
 (segment (start 106 106.5) (end 106 112.5) (width 0.25) (layer "F.Cu") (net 19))
 (segment (start 112.46 103.27) (end 112.46 102.54) (width 0.25) (layer "F.Cu") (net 19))
 (segment (start 109.23 103.27) (end 106 106.5) (width 0.25) (layer "F.Cu") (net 19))
 (segment (start 115 100) (end 121.69 100) (width 0.25) (layer "F.Cu") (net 19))
 (segment (start 112.46 102.54) (end 115 100) (width 0.25) (layer "F.Cu") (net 19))
 (segment (start 133 115) (end 138 120) (width 0.25) (layer "F.Cu") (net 19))
 (segment (start 124.96 103.27) (end 124.96 107.46) (width 0.25) (layer "F.Cu") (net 19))
 (segment (start 124.96 107.46) (end 132.5 115) (width 0.25) (layer "F.Cu") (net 19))
 (segment (start 112.46 103.27) (end 109.23 103.27) (width 0.25) (layer "F.Cu") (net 19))
 (segment (start 121.69 100) (end 124.96 103.27) (width 0.25) (layer "F.Cu") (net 19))
 (segment (start 145.08 85) (end 145 85) (width 0.25) (layer "F.Cu") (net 2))
 (segment (start 147.5 82.58) (end 145.08 85) (width 0.25) (layer "F.Cu") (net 2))
 (segment (start 145 95.16) (end 147.5 97.66) (width 0.25) (layer "F.Cu") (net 2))
 (segment (start 142.5 82.58) (end 147.5 82.58) (width 0.25) (layer "F.Cu") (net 2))
 (segment (start 140 120) (end 140 112.5) (width 0.25) (layer "F.Cu") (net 2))
 (segment (start 97.5 85) (end 102.5 80) (width 0.25) (layer "F.Cu") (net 2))
 (segment (start 102.5 80) (end 102.5 77.5) (width 0.25) (layer "F.Cu") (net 2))
 (segment (start 145 85) (end 145 95.16) (width 0.25) (layer "F.Cu") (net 2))
 (via (at 97.5 85) (size 0.8) (drill 0.4) (layers "F.Cu" "B.Cu") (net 2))
 (via (at 102.5 77.5) (size 0.8) (drill 0.4) (layers "F.Cu" "B.Cu") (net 2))
 (segment (start 120.77 103.27) (end 125 107.5) (width 0.25) (layer "B.Cu") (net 2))
 (segment (start 127.5 107.5) (end 130.04 104.96) (width 0.25) (layer "B.Cu") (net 2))
 (segment (start 117.54 103.27) (end 117.54 104.96) (width 0.25) (layer "B.Cu") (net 2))
 (segment (start 140 107.5) (end 137.5 107.5) (width 0.25) (layer "B.Cu") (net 2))
 (segment (start 140 110) (end 140 112.5) (width 0.25) (layer "B.Cu") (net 2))
 (segment (start 137.5 107.5) (end 140 110) (width 0.25) (layer "B.Cu") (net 2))
 (segment (start 135 107.5) (end 137.5 107.5) (width 0.25) (layer "B.Cu") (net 2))
 (segment (start 130.77 103.27) (end 135 107.5) (width 0.25) (layer "B.Cu") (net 2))
 (segment (start 142.5 105) (end 142.5 102.5) (width 0.25) (layer "B.Cu") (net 2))
 (segment (start 102.5 75) (end 102.3 74.8) (width 0.25) (layer "B.Cu") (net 2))
 (segment (start 115 107.5) (end 105 107.5) (width 0.25) (layer "B.Cu") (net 2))
 (segment (start 117.54 104.96) (end 115 107.5) (width 0.25) (layer "B.Cu") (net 2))
 (segment (start 130.04 103.27) (end 130.77 103.27) (width 0.25) (layer "B.Cu") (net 2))
 (segment (start 140 105) (end 142.5 102.5) (width 0.25) (layer "B.Cu") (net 2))
 (segment (start 147.5 97.66) (end 142.66 102.5) (width 0.25) (layer "B.Cu") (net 2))
 (segment (start 125 107.5) (end 127.5 107.5) (width 0.25) (layer "B.Cu") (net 2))
 (segment (start 102.3 72.5) (end 102.3 74.8) (width 0.25) (layer "B.Cu") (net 2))
 (segment (start 97.5 85) (end 97.5 110) (width 0.25) (layer "B.Cu") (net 2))
 (segment (start 117.54 103.27) (end 120.77 103.27) (width 0.25) (layer "B.Cu") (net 2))
 (segment (start 97.5 110) (end 100 112.5) (width 0.25) (layer "B.Cu") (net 2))
 (segment (start 105 107.5) (end 100 112.5) (width 0.25) (layer "B.Cu") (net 2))
 (segment (start 142.5 105) (end 140 107.5) (width 0.25) (layer "B.Cu") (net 2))
 (segment (start 102.5 77.5) (end 102.5 75) (width 0.25) (layer "B.Cu") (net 2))
 (segment (start 130.04 104.96) (end 130.04 103.27) (width 0.25) (layer "B.Cu") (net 2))
 (segment (start 144.96 102.54) (end 138 109.5) (width 0.25) (layer "F.Cu") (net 18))
 (segment (start 138 112.5) (end 135 112.5) (width 0.25) (layer "F.Cu") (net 18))
 (segment (start 135 112.5) (end 127.5 105) (width 0.25) (layer "F.Cu") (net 18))
 (segment (start 144.96 102.5) (end 144.96 102.54) (width 0.25) (layer "F.Cu") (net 18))
 (segment (start 127.5 105) (end 127.5 103.27) (width 0.25) (layer "F.Cu") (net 18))
 (segment (start 138 109.5) (end 138 112.5) (width 0.25) (layer "F.Cu") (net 18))
 (segment (start 135 92.5) (end 138 95.5) (width 0.25) (layer "B.Cu") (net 3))
 (segment (start 112.5 92.5) (end 135 92.5) (width 0.25) (layer "B.Cu") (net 3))
 (segment (start 138 103) (end 138 105) (width 0.25) (layer "B.Cu") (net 3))
 (segment (start 117.5 100) (end 135 100) (width 0.25) (layer "B.Cu") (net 3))
 (segment (start 115 102.5) (end 117.5 100) (width 0.25) (layer "B.Cu") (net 3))
 (segment (start 99.76 79.76) (end 112.5 92.5) (width 0.25) (layer "B.Cu") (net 3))
 (segment (start 138 95.5) (end 138 103) (width 0.25) (layer "B.Cu") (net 3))
 (segment (start 135 100) (end 138 103) (width 0.25) (layer "B.Cu") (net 3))
 (segment (start 115 103.27) (end 115 102.5) (width 0.25) (layer "B.Cu") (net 3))
 (segment (start 99.76 72.5) (end 99.76 79.76) (width 0.25) (layer "B.Cu") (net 3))
 (segment (start 147.5 102.5) (end 147.5 112.5) (width 0.25) (layer "F.Cu") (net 35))
 (segment (start 147.5 72.42) (end 150 74.92) (width 0.25) (layer "F.Cu") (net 1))
 (segment (start 150 85) (end 147.5 87.5) (width 0.25) (layer "F.Cu") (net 1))
 (segment (start 150 74.92) (end 150 85) (width 0.25) (layer "F.Cu") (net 1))
 (segment (start 142.5 72.42) (end 147.5 72.42) (width 0.25) (layer "F.Cu") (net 1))
 (segment (start 150 117.5) (end 150 90) (width 0.25) (layer "B.Cu") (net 1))
 (segment (start 150 90) (end 147.5 87.5) (width 0.25) (layer "B.Cu") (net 1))
 (segment (start 147.5 117.5) (end 150 117.5) (width 0.25) (layer "B.Cu") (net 1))
 (segment (start 144.84 100) (end 142.5 97.66) (width 0.25) (layer "F.Cu") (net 17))
 (segment (start 145 100) (end 144.84 100) (width 0.25) (layer "F.Cu") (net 17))
 (segment (start 146.23 102.5) (end 146.23 101.23) (width 0.25) (layer "F.Cu") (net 17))
 (segment (start 146.23 101.23) (end 145 100) (width 0.25) (layer "F.Cu") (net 17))
 (segment (start 137.62 87.5) (end 142.5 87.5) (width 0.25) (layer "F.Cu") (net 11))
 (segment (start 122.62 72.5) (end 137.62 87.5) (width 0.25) (layer "F.Cu") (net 11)))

